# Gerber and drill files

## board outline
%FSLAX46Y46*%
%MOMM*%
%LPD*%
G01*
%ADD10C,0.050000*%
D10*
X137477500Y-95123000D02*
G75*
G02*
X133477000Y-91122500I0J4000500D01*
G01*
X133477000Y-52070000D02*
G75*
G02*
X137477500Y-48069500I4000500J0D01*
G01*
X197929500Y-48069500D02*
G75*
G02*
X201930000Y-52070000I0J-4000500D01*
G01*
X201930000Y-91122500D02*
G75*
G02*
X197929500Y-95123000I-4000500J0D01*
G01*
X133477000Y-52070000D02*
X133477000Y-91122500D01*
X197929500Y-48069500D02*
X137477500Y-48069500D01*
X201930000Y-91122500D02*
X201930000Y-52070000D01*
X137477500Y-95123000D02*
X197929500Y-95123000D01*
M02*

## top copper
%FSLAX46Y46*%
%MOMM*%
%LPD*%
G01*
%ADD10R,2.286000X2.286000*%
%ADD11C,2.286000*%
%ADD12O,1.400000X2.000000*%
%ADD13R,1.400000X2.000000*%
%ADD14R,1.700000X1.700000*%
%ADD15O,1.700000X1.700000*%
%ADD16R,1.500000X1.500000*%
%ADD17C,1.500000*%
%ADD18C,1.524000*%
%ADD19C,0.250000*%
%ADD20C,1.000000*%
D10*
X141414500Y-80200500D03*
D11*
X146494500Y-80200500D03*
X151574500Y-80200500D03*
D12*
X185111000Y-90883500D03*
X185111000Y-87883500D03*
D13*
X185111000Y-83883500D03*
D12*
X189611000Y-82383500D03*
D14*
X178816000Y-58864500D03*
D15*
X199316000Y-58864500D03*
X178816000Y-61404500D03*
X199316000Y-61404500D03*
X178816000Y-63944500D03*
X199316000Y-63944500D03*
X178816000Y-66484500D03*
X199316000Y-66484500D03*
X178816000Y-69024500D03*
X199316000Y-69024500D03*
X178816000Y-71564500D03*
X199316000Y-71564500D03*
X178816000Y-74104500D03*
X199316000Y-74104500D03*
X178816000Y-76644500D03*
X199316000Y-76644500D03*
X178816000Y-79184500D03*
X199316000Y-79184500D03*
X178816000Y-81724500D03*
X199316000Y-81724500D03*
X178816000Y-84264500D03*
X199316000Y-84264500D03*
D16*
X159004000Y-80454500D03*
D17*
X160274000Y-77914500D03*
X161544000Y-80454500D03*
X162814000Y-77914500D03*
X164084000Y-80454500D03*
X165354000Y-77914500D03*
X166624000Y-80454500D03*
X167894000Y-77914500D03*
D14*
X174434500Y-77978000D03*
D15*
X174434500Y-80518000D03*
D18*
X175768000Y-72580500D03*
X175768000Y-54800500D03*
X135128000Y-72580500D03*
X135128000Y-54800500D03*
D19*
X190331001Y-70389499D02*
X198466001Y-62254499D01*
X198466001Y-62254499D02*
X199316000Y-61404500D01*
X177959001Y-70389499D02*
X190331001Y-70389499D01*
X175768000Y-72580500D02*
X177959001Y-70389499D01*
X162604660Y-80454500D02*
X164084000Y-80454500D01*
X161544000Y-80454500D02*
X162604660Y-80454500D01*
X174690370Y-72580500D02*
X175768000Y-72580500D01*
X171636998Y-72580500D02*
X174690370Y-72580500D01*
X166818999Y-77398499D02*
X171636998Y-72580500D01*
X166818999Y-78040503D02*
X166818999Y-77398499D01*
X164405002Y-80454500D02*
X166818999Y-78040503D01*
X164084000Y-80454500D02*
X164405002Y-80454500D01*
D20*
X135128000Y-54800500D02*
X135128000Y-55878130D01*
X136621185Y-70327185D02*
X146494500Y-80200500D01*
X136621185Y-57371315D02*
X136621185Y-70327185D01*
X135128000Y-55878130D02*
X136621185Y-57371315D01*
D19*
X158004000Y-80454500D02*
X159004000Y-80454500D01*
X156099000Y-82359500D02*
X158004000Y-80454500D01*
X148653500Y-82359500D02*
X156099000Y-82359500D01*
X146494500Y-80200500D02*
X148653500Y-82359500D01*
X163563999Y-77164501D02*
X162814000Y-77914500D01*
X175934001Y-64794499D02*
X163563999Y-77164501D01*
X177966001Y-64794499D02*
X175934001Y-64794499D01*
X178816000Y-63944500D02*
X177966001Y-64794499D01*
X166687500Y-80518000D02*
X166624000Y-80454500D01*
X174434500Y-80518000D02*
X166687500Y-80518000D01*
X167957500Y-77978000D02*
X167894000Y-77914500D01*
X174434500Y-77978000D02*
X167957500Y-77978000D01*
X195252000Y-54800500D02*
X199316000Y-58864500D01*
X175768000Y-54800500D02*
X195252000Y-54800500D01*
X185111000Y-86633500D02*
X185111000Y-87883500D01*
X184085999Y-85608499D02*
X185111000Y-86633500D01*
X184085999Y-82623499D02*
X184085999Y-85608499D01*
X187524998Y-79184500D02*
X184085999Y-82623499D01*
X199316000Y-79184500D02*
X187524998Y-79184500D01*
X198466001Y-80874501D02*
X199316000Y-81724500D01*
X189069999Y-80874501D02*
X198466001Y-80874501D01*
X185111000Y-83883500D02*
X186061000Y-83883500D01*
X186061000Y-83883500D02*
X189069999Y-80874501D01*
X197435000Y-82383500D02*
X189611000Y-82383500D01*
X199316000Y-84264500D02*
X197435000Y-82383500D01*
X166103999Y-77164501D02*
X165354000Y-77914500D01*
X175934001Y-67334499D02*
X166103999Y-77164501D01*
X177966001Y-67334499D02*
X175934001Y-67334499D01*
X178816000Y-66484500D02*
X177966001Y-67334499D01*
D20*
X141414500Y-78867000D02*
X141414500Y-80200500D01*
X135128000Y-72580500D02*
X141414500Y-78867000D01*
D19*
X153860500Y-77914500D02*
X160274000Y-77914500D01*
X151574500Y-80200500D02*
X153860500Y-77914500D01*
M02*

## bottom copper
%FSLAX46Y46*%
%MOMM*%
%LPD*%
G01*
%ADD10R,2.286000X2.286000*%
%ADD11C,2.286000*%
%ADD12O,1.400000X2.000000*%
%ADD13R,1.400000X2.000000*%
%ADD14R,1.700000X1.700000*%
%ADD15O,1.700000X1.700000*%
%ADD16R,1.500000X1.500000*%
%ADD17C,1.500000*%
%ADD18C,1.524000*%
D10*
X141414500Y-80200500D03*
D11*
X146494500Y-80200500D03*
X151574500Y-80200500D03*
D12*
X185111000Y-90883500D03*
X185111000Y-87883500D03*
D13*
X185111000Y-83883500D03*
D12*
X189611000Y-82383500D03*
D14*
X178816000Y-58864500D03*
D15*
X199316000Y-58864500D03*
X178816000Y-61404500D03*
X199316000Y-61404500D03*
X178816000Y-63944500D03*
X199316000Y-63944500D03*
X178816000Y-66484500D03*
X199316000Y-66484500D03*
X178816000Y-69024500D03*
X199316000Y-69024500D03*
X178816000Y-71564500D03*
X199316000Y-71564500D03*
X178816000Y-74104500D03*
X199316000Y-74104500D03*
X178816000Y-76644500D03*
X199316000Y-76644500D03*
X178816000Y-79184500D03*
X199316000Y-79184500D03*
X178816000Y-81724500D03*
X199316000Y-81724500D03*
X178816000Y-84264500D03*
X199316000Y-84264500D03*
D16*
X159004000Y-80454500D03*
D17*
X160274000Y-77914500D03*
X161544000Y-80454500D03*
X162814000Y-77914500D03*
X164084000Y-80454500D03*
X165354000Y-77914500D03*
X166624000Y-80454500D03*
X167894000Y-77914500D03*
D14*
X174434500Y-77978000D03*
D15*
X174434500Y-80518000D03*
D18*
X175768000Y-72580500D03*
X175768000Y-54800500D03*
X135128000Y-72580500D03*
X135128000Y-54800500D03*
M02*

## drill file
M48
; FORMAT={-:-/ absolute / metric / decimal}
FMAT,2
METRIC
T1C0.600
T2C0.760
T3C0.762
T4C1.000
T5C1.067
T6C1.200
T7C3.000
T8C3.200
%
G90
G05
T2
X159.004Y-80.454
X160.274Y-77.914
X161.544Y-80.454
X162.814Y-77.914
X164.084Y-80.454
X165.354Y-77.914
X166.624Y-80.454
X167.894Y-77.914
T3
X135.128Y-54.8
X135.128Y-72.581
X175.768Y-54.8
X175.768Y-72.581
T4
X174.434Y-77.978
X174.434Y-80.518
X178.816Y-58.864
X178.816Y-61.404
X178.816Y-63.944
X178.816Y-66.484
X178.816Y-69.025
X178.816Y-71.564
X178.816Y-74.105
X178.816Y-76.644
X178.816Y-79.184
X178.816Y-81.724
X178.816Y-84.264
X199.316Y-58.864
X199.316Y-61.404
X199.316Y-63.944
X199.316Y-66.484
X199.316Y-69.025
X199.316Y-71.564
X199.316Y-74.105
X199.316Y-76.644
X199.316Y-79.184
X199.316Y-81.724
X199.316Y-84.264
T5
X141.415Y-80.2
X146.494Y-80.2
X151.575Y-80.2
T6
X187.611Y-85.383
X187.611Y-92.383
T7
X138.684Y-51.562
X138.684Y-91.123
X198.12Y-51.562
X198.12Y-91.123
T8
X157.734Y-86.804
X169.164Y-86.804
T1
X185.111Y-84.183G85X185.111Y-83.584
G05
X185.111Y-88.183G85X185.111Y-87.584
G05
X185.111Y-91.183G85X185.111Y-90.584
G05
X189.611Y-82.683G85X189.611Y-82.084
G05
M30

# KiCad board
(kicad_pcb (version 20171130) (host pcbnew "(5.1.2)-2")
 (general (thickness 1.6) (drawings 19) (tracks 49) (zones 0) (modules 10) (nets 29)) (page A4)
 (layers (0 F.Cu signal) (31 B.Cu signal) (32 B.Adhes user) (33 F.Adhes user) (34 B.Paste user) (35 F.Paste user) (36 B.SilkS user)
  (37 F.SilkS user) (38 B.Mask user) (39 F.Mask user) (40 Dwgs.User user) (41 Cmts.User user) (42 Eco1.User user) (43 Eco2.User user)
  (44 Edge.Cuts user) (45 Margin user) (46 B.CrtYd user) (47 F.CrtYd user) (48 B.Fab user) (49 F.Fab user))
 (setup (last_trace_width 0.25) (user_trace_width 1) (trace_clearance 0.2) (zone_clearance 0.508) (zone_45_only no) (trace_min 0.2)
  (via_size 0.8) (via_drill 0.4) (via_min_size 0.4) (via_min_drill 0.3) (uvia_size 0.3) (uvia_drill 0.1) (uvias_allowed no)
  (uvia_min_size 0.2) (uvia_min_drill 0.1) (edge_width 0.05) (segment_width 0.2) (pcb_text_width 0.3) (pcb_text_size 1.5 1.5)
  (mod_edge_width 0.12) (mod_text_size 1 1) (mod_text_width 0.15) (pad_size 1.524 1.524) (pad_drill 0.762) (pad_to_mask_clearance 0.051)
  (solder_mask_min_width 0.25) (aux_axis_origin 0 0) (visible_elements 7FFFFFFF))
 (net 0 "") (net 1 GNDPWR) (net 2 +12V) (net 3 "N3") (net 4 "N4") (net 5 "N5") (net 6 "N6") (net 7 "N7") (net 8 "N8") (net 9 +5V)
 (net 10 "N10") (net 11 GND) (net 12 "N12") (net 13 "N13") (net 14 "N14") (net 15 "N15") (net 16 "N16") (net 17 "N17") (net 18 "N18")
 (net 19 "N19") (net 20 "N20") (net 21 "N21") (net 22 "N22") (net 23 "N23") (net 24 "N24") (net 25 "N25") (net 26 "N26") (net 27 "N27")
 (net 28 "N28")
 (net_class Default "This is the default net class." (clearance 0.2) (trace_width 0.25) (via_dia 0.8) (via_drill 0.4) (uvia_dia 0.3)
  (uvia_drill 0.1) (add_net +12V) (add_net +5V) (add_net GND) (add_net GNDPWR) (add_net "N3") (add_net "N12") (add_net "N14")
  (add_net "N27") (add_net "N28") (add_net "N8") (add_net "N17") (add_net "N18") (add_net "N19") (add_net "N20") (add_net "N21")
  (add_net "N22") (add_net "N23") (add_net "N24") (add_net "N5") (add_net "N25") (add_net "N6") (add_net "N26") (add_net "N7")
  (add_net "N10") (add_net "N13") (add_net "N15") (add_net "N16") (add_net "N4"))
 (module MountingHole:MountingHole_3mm (layer F.Cu) (at 138.684 51.562)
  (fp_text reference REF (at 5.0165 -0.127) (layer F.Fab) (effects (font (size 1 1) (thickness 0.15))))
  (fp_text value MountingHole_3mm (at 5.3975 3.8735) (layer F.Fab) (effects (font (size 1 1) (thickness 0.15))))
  (pad 1 np_thru_hole circle (at 0 0) (size 3 3) (drill 3) (layers *.Cu *.Mask)))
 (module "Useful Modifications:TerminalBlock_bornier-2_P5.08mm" (layer F.Cu) (at 141.4145 80.2005)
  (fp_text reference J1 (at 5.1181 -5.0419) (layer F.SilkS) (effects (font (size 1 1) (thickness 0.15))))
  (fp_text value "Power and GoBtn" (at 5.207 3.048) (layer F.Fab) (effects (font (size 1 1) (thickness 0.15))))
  (pad 1 thru_hole rect (at 0 0) (size 2.286 2.286) (drill 1.0668) (layers *.Cu *.Mask) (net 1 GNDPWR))
  (pad 2 thru_hole circle (at 5.08 0) (size 2.286 2.286) (drill 1.0668) (layers *.Cu *.Mask) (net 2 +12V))
  (pad 3 thru_hole circle (at 10.16 0) (size 2.286 2.286) (drill 1.0668) (layers *.Cu *.Mask) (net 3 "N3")))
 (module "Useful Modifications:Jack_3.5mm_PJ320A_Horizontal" (layer F.Cu) (at 189.611 83.8835 180)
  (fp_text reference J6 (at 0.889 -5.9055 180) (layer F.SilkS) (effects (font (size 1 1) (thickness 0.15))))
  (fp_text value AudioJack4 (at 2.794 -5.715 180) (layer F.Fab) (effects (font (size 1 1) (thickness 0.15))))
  (pad "" np_thru_hole circle (at 2 -1.5 90) (size 1.2 1.2) (drill 1.2) (layers *.Cu *.Mask))
  (pad "" np_thru_hole circle (at 2 -8.5 90) (size 1.2 1.2) (drill 1.2) (layers *.Cu *.Mask))
  (pad R2 thru_hole oval (at 4.5 -7 90) (size 2 1.4) (drill oval 1.2 0.6) (layers *.Cu *.Mask) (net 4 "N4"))
  (pad R1 thru_hole oval (at 4.5 -4 90) (size 2 1.4) (drill oval 1.2 0.6) (layers *.Cu *.Mask) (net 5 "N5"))
  (pad T thru_hole rect (at 4.5 0 90) (size 2 1.4) (drill oval 1.2 0.6) (layers *.Cu *.Mask) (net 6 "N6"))
  (pad S thru_hole oval (at 0 1.5 90) (size 2 1.4) (drill oval 1.2 0.6) (layers *.Cu *.Mask) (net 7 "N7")))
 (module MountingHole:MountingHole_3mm (layer F.Cu) (at 198.12 51.562)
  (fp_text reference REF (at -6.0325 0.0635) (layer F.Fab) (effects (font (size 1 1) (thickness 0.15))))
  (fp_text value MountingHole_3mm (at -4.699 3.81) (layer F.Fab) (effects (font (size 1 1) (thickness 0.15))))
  (pad 1 np_thru_hole circle (at 0 0) (size 3 3) (drill 3) (layers *.Cu *.Mask)))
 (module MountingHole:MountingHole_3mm (layer F.Cu) (at 198.12 91.1225)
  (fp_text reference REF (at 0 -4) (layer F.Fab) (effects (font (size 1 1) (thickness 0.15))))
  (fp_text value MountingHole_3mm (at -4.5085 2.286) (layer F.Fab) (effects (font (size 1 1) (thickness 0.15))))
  (pad 1 np_thru_hole circle (at 0 0) (size 3 3) (drill 3) (layers *.Cu *.Mask)))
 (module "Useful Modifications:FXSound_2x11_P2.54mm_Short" (layer F.Cu) (at 178.816 58.8645)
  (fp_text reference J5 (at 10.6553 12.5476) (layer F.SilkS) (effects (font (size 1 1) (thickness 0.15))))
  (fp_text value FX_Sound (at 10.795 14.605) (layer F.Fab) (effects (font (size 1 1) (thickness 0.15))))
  (pad 1 thru_hole rect (at 0 0) (size 1.7 1.7) (drill 1) (layers *.Cu *.Mask) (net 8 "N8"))
  (pad 2 thru_hole oval (at 20.5 0) (size 1.7 1.7) (drill 1) (layers *.Cu *.Mask) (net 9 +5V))
  (pad 3 thru_hole oval (at 0 2.54) (size 1.7 1.7) (drill 1) (layers *.Cu *.Mask) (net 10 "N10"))
  (pad 4 thru_hole oval (at 20.5 2.54) (size 1.7 1.7) (drill 1) (layers *.Cu *.Mask) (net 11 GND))
  (pad 5 thru_hole oval (at 0 5.08) (size 1.7 1.7) (drill 1) (layers *.Cu *.Mask) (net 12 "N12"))
  (pad 6 thru_hole oval (at 20.5 5.08) (size 1.7 1.7) (drill 1) (layers *.Cu *.Mask) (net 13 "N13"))
  (pad 7 thru_hole oval (at 0 7.62) (size 1.7 1.7) (drill 1) (layers *.Cu *.Mask) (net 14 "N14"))
  (pad 8 thru_hole oval (at 20.5 7.62) (size 1.7 1.7) (drill 1) (layers *.Cu *.Mask) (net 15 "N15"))
  (pad 9 thru_hole oval (at 0 10.16) (size 1.7 1.7) (drill 1) (layers *.Cu *.Mask) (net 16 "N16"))
  (pad 10 thru_hole oval (at 20.5 10.16) (size 1.7 1.7) (drill 1) (layers *.Cu *.Mask) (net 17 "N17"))
  (pad 11 thru_hole oval (at 0 12.7) (size 1.7 1.7) (drill 1) (layers *.Cu *.Mask) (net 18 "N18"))
  (pad 12 thru_hole oval (at 20.5 12.7) (size 1.7 1.7) (drill 1) (layers *.Cu *.Mask) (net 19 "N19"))
  (pad 13 thru_hole oval (at 0 15.24) (size 1.7 1.7) (drill 1) (layers *.Cu *.Mask) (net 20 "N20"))
  (pad 14 thru_hole oval (at 20.5 15.24) (size 1.7 1.7) (drill 1) (layers *.Cu *.Mask) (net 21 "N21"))
  (pad 15 thru_hole oval (at 0 17.78) (size 1.7 1.7) (drill 1) (layers *.Cu *.Mask) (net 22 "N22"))
  (pad 16 thru_hole oval (at 20.5 17.78) (size 1.7 1.7) (drill 1) (layers *.Cu *.Mask) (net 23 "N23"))
  (pad 17 thru_hole oval (at 0 20.32) (size 1.7 1.7) (drill 1) (layers *.Cu *.Mask) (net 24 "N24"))
  (pad 18 thru_hole oval (at 20.5 20.32) (size 1.7 1.7) (drill 1) (layers *.Cu *.Mask) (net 5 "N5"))
  (pad 19 thru_hole oval (at 0 22.86) (size 1.7 1.7) (drill 1) (layers *.Cu *.Mask) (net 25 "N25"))
  (pad 20 thru_hole oval (at 20.5 22.86) (size 1.7 1.7) (drill 1) (layers *.Cu *.Mask) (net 6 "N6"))
  (pad 21 thru_hole oval (at 0 25.4) (size 1.7 1.7) (drill 1) (layers *.Cu *.Mask) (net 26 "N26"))
  (pad 22 thru_hole oval (at 20.5 25.4) (size 1.7 1.7) (drill 1) (layers *.Cu *.Mask) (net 7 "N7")))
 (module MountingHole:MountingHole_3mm (layer F.Cu) (at 138.684 91.1225)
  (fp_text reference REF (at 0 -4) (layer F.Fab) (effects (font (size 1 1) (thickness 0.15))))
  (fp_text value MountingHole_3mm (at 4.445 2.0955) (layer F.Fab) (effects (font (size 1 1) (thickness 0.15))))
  (pad 1 np_thru_hole circle (at 0 0) (size 3 3) (drill 3) (layers *.Cu *.Mask)))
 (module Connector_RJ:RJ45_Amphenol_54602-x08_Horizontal (layer F.Cu) (at 159.004 80.4545)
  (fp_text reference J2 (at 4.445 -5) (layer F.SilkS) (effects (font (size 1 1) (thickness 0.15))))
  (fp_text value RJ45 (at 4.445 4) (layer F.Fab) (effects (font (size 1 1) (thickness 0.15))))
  (pad "" np_thru_hole circle (at 10.16 6.35) (size 3.2 3.2) (drill 3.2) (layers *.Cu *.Mask))
  (pad "" np_thru_hole circle (at -1.27 6.35) (size 3.2 3.2) (drill 3.2) (layers *.Cu *.Mask))
  (pad 1 thru_hole rect (at 0 0) (size 1.5 1.5) (drill 0.76) (layers *.Cu *.Mask) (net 2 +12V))
  (pad 2 thru_hole circle (at 1.27 -2.54) (size 1.5 1.5) (drill 0.76) (layers *.Cu *.Mask) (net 3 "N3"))
  (pad 3 thru_hole circle (at 2.54 0) (size 1.5 1.5) (drill 0.76) (layers *.Cu *.Mask) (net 11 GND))
  (pad 4 thru_hole circle (at 3.81 -2.54) (size 1.5 1.5) (drill 0.76) (layers *.Cu *.Mask) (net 12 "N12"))
  (pad 5 thru_hole circle (at 5.08 0) (size 1.5 1.5) (drill 0.76) (layers *.Cu *.Mask) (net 11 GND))
  (pad 6 thru_hole circle (at 6.35 -2.54) (size 1.5 1.5) (drill 0.76) (layers *.Cu *.Mask) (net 14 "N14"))
  (pad 7 thru_hole circle (at 7.62 0) (size 1.5 1.5) (drill 0.76) (layers *.Cu *.Mask) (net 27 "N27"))
  (pad 8 thru_hole circle (at 8.89 -2.54) (size 1.5 1.5) (drill 0.76) (layers *.Cu *.Mask) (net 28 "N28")))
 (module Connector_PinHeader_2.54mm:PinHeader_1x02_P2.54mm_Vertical (layer F.Cu) (at 174.4345 77.978)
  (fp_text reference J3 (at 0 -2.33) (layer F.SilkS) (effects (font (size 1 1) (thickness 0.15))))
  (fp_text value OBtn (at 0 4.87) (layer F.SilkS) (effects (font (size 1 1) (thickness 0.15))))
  (pad 1 thru_hole rect (at 0 0) (size 1.7 1.7) (drill 1) (layers *.Cu *.Mask) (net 28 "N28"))
  (pad 2 thru_hole oval (at 0 2.54) (size 1.7 1.7) (drill 1) (layers *.Cu *.Mask) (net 27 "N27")))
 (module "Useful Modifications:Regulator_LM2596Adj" (layer F.Cu) (at 157.988 64.9605)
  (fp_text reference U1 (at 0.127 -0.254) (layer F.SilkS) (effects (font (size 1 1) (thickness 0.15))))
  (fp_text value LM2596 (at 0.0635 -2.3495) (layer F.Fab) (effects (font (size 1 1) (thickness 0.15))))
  (pad 6 thru_hole circle (at 17.78 7.62) (size 1.524 1.524) (drill 0.762) (layers *.Cu *.Mask) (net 11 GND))
  (pad 4 thru_hole circle (at 17.78 -10.16) (size 1.524 1.524) (drill 0.762) (layers *.Cu *.Mask) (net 9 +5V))
  (pad 1 thru_hole circle (at -22.86 7.62) (size 1.524 1.524) (drill 0.762) (layers *.Cu *.Mask) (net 1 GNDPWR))
  (pad 2 thru_hole circle (at -22.86 -10.16) (size 1.524 1.524) (drill 0.762) (layers *.Cu *.Mask) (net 2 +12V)))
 (gr_arc (start 137.4775 91.1225) (end 133.477 91.1225) (angle -90) (layer Edge.Cuts) (width 0.05))
 (gr_arc (start 137.4775 52.07) (end 137.4775 48.0695) (angle -90) (layer Edge.Cuts) (width 0.05))
 (gr_arc (start 197.9295 52.07) (end 201.93 52.07) (angle -90) (layer Edge.Cuts) (width 0.05))
 (gr_arc (start 197.9295 91.1225) (end 197.9295 95.123) (angle -90) (layer Edge.Cuts) (width 0.05))
 (gr_line (start 133.477 52.07) (end 133.477 91.1225) (layer Edge.Cuts) (width 0.05))
 (gr_line (start 197.9295 48.0695) (end 137.4775 48.0695) (layer Edge.Cuts) (width 0.05))
 (gr_line (start 201.93 91.1225) (end 201.93 52.07) (layer Edge.Cuts) (width 0.05))
 (gr_line (start 137.4775 95.123) (end 197.9295 95.123) (layer Edge.Cuts) (width 0.05))
 (segment (start 190.331001 70.389499) (end 198.466001 62.254499) (width 0.25) (layer F.Cu) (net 11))
 (segment (start 198.466001 62.254499) (end 199.316 61.4045) (width 0.25) (layer F.Cu) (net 11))
 (segment (start 177.959001 70.389499) (end 190.331001 70.389499) (width 0.25) (layer F.Cu) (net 11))
 (segment (start 175.768 72.5805) (end 177.959001 70.389499) (width 0.25) (layer F.Cu) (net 11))
 (segment (start 162.60466 80.4545) (end 164.084 80.4545) (width 0.25) (layer F.Cu) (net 11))
 (segment (start 161.544 80.4545) (end 162.60466 80.4545) (width 0.25) (layer F.Cu) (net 11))
 (segment (start 174.69037 72.5805) (end 175.768 72.5805) (width 0.25) (layer F.Cu) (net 11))
 (segment (start 171.636998 72.5805) (end 174.69037 72.5805) (width 0.25) (layer F.Cu) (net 11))
 (segment (start 166.818999 77.398499) (end 171.636998 72.5805) (width 0.25) (layer F.Cu) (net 11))
 (segment (start 166.818999 78.040503) (end 166.818999 77.398499) (width 0.25) (layer F.Cu) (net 11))
 (segment (start 164.405002 80.4545) (end 166.818999 78.040503) (width 0.25) (layer F.Cu) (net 11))
 (segment (start 164.084 80.4545) (end 164.405002 80.4545) (width 0.25) (layer F.Cu) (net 11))
 (segment (start 135.128 54.8005) (end 135.128 55.87813) (width 1) (layer F.Cu) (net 2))
 (segment (start 136.621185 70.327185) (end 146.4945 80.2005) (width 1) (layer F.Cu) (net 2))
 (segment (start 136.621185 57.371315) (end 136.621185 70.327185) (width 1) (layer F.Cu) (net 2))
 (segment (start 135.128 55.87813) (end 136.621185 57.371315) (width 1) (layer F.Cu) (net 2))
 (segment (start 158.004 80.4545) (end 159.004 80.4545) (width 0.25) (layer F.Cu) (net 2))
 (segment (start 156.099 82.3595) (end 158.004 80.4545) (width 0.25) (layer F.Cu) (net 2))
 (segment (start 148.6535 82.3595) (end 156.099 82.3595) (width 0.25) (layer F.Cu) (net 2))
 (segment (start 146.4945 80.2005) (end 148.6535 82.3595) (width 0.25) (layer F.Cu) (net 2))
 (segment (start 163.563999 77.164501) (end 162.814 77.9145) (width 0.25) (layer F.Cu) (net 12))
 (segment (start 175.934001 64.794499) (end 163.563999 77.164501) (width 0.25) (layer F.Cu) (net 12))
 (segment (start 177.966001 64.794499) (end 175.934001 64.794499) (width 0.25) (layer F.Cu) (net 12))
 (segment (start 178.816 63.9445) (end 177.966001 64.794499) (width 0.25) (layer F.Cu) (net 12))
 (segment (start 166.6875 80.518) (end 166.624 80.4545) (width 0.25) (layer F.Cu) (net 27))
 (segment (start 174.4345 80.518) (end 166.6875 80.518) (width 0.25) (layer F.Cu) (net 27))
 (segment (start 167.9575 77.978) (end 167.894 77.9145) (width 0.25) (layer F.Cu) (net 28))
 (segment (start 174.4345 77.978) (end 167.9575 77.978) (width 0.25) (layer F.Cu) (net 28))
 (segment (start 195.252 54.8005) (end 199.316 58.8645) (width 0.25) (layer F.Cu) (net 9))
 (segment (start 175.768 54.8005) (end 195.252 54.8005) (width 0.25) (layer F.Cu) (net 9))
 (segment (start 185.111 86.6335) (end 185.111 87.8835) (width 0.25) (layer F.Cu) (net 5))
 (segment (start 184.085999 85.608499) (end 185.111 86.6335) (width 0.25) (layer F.Cu) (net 5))
 (segment (start 184.085999 82.623499) (end 184.085999 85.608499) (width 0.25) (layer F.Cu) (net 5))
 (segment (start 187.524998 79.1845) (end 184.085999 82.623499) (width 0.25) (layer F.Cu) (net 5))
 (segment (start 199.316 79.1845) (end 187.524998 79.1845) (width 0.25) (layer F.Cu) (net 5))
 (segment (start 198.466001 80.874501) (end 199.316 81.7245) (width 0.25) (layer F.Cu) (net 6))
 (segment (start 189.069999 80.874501) (end 198.466001 80.874501) (width 0.25) (layer F.Cu) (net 6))
 (segment (start 185.111 83.8835) (end 186.061 83.8835) (width 0.25) (layer F.Cu) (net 6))
 (segment (start 186.061 83.8835) (end 189.069999 80.874501) (width 0.25) (layer F.Cu) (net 6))
 (segment (start 197.435 82.3835) (end 189.611 82.3835) (width 0.25) (layer F.Cu) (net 7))
 (segment (start 199.316 84.2645) (end 197.435 82.3835) (width 0.25) (layer F.Cu) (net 7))
 (segment (start 166.103999 77.164501) (end 165.354 77.9145) (width 0.25) (layer F.Cu) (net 14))
 (segment (start 175.934001 67.334499) (end 166.103999 77.164501) (width 0.25) (layer F.Cu) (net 14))
 (segment (start 177.966001 67.334499) (end 175.934001 67.334499) (width 0.25) (layer F.Cu) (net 14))
 (segment (start 178.816 66.4845) (end 177.966001 67.334499) (width 0.25) (layer F.Cu) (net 14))
 (segment (start 141.4145 78.867) (end 141.4145 80.2005) (width 1) (layer F.Cu) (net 1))
 (segment (start 135.128 72.5805) (end 141.4145 78.867) (width 1) (layer F.Cu) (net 1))
 (segment (start 153.8605 77.9145) (end 160.274 77.9145) (width 0.25) (layer F.Cu) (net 3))
 (segment (start 151.5745 80.2005) (end 153.8605 77.9145) (width 0.25) (layer F.Cu) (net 3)))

